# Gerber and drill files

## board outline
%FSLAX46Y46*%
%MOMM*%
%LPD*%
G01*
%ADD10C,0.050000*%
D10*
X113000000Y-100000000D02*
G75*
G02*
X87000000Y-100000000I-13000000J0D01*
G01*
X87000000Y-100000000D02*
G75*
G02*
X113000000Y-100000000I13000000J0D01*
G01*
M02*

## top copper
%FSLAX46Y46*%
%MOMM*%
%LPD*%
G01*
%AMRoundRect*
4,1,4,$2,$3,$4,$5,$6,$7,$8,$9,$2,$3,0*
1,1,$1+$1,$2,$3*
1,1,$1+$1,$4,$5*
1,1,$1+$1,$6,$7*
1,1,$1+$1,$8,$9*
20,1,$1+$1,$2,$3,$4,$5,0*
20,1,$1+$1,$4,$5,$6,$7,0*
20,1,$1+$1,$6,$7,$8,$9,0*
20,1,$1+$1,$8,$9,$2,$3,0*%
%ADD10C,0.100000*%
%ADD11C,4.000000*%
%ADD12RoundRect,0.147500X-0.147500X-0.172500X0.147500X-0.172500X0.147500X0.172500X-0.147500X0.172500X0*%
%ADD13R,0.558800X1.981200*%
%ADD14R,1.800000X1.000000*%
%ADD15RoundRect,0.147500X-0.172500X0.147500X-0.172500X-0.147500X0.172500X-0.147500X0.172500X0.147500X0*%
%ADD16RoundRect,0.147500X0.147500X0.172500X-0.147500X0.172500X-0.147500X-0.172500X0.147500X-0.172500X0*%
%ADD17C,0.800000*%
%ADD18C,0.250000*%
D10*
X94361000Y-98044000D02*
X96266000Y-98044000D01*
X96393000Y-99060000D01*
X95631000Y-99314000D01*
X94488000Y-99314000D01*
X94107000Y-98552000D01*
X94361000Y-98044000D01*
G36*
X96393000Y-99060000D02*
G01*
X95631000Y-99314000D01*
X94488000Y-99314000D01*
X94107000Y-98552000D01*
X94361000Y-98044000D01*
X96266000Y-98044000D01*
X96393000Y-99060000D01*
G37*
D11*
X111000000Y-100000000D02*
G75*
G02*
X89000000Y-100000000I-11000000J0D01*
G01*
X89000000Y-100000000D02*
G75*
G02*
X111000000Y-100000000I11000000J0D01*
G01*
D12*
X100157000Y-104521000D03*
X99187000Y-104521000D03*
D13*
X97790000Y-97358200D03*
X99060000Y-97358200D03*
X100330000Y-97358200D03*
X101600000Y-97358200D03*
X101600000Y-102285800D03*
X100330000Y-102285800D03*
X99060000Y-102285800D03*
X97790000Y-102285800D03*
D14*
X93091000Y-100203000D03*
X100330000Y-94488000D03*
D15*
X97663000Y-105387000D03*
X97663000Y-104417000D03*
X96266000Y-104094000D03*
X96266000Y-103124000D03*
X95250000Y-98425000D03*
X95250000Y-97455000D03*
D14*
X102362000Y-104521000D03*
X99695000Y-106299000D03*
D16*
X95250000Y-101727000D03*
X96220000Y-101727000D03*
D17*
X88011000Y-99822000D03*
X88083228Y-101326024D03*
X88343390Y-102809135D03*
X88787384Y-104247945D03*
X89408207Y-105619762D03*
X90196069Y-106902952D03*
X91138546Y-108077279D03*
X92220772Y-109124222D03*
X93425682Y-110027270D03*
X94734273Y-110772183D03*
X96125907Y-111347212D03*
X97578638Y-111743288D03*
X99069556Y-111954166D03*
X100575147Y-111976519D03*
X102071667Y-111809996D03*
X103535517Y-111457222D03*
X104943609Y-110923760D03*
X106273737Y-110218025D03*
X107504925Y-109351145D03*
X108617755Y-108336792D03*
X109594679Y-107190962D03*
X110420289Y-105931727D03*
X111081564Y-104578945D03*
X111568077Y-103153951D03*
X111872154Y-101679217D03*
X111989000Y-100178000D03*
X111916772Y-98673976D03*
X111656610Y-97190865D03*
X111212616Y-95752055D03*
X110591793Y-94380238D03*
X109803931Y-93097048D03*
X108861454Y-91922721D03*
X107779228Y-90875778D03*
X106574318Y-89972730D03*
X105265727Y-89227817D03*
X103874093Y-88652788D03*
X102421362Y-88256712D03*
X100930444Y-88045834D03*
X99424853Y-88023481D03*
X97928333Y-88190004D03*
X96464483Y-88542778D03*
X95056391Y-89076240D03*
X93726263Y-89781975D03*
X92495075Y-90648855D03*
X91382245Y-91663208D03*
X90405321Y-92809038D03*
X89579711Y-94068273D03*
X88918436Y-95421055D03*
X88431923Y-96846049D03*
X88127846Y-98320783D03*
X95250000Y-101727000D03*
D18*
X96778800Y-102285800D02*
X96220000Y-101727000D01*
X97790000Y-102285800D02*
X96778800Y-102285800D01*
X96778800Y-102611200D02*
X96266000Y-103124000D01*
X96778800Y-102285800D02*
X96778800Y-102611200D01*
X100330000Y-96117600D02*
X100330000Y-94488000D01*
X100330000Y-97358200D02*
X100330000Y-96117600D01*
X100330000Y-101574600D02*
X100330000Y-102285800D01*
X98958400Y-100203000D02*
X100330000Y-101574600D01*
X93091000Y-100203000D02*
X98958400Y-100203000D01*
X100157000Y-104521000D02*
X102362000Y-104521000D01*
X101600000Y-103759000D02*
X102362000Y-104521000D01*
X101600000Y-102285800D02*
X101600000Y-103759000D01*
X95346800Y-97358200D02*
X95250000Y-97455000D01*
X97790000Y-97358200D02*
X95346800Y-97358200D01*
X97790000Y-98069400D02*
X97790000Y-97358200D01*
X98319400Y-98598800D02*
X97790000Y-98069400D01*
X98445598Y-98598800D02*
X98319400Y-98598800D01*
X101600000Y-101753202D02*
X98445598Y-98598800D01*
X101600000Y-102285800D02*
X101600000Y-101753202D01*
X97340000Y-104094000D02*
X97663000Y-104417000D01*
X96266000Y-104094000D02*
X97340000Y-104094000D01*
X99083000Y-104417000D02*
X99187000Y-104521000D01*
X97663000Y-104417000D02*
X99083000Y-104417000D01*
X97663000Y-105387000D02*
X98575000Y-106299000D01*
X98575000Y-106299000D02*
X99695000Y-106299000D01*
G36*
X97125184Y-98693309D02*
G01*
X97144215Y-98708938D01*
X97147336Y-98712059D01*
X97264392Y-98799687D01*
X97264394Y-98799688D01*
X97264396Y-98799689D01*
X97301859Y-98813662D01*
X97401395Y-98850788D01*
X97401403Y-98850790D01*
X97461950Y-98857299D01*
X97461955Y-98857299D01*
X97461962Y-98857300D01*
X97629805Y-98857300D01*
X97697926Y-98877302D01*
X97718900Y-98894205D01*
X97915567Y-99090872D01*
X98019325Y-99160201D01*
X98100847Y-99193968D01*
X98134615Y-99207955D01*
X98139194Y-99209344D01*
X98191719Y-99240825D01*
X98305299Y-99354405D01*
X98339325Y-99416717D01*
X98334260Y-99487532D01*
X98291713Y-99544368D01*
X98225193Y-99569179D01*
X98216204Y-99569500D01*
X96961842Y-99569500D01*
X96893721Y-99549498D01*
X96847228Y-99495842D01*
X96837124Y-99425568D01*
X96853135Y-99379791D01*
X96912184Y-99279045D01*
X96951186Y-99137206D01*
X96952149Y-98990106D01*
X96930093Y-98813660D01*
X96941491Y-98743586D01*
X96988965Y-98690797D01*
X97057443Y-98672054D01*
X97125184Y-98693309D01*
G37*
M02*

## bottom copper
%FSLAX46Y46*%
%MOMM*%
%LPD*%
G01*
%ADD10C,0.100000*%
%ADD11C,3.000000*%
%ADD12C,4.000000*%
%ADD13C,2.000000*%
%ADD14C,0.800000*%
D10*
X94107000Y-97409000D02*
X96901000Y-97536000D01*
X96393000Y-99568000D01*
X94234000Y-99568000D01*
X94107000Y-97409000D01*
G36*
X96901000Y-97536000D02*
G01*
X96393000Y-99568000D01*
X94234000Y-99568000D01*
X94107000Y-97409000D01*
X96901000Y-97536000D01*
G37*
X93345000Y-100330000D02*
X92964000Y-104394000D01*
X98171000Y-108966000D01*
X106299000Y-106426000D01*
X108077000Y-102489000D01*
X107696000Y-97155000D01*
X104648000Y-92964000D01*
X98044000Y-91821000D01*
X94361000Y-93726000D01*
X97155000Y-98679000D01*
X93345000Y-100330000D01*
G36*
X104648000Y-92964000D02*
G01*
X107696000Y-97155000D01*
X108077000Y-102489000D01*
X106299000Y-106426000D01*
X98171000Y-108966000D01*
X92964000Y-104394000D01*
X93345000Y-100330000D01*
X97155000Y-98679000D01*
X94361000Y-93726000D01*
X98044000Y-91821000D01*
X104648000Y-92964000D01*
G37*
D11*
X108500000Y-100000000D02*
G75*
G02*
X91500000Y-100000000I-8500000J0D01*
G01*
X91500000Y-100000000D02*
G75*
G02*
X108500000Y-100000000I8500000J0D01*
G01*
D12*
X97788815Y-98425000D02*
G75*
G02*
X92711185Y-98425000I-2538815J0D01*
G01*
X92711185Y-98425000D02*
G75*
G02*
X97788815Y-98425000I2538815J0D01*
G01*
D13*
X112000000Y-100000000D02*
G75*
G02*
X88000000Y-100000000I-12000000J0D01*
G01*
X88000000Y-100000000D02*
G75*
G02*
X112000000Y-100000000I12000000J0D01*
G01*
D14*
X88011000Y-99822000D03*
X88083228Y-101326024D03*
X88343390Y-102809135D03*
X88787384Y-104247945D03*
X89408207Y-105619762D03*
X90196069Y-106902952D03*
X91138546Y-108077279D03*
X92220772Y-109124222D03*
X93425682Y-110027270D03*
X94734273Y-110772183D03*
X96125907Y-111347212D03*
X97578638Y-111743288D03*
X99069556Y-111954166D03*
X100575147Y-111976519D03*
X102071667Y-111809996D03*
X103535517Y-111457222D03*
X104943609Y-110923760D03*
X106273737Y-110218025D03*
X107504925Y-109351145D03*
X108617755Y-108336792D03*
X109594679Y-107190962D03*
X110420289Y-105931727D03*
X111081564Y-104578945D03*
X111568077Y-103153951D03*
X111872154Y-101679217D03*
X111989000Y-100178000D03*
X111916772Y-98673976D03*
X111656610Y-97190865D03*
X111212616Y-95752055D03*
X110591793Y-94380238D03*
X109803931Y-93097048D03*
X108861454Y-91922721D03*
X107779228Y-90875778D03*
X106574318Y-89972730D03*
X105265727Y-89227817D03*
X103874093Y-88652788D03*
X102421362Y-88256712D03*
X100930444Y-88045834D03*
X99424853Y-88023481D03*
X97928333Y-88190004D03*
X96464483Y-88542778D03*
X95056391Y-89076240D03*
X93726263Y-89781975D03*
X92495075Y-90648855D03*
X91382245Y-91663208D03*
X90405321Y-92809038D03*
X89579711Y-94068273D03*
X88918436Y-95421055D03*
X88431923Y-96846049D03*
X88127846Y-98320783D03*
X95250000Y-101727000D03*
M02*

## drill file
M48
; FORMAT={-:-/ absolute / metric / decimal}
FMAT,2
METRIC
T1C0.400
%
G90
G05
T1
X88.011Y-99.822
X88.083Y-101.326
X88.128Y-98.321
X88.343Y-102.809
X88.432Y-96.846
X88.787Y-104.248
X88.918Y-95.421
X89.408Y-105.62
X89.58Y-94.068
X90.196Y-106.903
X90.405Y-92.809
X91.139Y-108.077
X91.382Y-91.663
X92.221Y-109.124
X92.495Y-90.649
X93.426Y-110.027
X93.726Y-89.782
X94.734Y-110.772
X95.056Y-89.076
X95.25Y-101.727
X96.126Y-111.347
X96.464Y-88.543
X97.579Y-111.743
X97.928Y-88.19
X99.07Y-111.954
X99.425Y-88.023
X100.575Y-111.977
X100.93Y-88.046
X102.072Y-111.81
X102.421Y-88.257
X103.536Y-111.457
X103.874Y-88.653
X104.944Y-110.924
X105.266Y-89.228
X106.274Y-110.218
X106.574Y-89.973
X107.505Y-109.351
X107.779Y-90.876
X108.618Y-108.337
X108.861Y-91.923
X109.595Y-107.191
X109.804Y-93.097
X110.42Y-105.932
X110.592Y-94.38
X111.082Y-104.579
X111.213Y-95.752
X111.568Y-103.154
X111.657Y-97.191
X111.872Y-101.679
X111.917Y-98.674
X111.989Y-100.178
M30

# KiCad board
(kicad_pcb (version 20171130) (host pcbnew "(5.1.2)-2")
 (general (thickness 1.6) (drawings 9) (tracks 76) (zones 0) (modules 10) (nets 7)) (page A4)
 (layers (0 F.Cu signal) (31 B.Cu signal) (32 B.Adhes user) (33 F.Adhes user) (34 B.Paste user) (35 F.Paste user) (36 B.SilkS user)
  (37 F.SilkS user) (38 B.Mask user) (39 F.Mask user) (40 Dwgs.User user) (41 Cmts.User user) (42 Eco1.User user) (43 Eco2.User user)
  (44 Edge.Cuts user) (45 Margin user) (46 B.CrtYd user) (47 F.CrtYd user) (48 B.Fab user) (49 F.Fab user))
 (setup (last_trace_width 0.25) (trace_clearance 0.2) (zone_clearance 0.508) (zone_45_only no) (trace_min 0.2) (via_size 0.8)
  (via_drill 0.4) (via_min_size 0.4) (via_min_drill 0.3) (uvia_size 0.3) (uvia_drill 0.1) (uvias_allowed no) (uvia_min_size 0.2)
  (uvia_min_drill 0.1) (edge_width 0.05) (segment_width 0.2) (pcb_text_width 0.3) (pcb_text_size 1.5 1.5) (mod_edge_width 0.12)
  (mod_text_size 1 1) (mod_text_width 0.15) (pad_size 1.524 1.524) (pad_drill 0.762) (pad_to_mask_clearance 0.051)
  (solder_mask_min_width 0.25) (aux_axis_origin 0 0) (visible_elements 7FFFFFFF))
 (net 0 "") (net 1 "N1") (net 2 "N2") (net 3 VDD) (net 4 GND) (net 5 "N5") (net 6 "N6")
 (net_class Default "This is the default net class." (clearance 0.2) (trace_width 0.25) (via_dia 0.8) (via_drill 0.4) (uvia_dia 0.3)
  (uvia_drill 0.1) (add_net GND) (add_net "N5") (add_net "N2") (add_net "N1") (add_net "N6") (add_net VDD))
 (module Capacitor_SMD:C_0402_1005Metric (layer F.Cu) (at 99.672 104.521)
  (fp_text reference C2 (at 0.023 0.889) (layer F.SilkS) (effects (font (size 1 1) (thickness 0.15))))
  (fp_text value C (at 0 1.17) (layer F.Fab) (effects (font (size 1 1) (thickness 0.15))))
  (pad 2 smd roundrect (at 0.485 0) (size 0.59 0.64) (layers F.Cu F.Paste F.Mask) (roundrect_rratio 0.25) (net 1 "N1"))
  (pad 1 smd roundrect (at -0.485 0) (size 0.59 0.64) (layers F.Cu F.Paste F.Mask) (roundrect_rratio 0.25) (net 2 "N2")))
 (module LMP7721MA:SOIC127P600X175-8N (layer F.Cu) (at 99.695 99.822 90)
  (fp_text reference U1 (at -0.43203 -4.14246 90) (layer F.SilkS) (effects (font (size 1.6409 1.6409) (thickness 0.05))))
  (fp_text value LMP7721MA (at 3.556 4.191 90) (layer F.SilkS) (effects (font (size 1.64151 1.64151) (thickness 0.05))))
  (pad 8 smd rect (at 2.4638 -1.905 90) (size 1.9812 0.5588) (layers F.Cu F.Paste F.Mask) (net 1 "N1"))
  (pad 7 smd rect (at 2.4638 -0.635 90) (size 1.9812 0.5588) (layers F.Cu F.Paste F.Mask))
  (pad 6 smd rect (at 2.4638 0.635 90) (size 1.9812 0.5588) (layers F.Cu F.Paste F.Mask) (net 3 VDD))
  (pad 5 smd rect (at 2.4638 1.905 90) (size 1.9812 0.5588) (layers F.Cu F.Paste F.Mask))
  (pad 4 smd rect (at -2.4638 1.905 90) (size 1.9812 0.5588) (layers F.Cu F.Paste F.Mask) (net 1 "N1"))
  (pad 3 smd rect (at -2.4638 0.635 90) (size 1.9812 0.5588) (layers F.Cu F.Paste F.Mask) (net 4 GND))
  (pad 2 smd rect (at -2.4638 -0.635 90) (size 1.9812 0.5588) (layers F.Cu F.Paste F.Mask))
  (pad 1 smd rect (at -2.4638 -1.905 90) (size 1.9812 0.5588) (layers F.Cu F.Paste F.Mask) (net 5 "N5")))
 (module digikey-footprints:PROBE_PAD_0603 (layer F.Cu) (at 93.091 100.203)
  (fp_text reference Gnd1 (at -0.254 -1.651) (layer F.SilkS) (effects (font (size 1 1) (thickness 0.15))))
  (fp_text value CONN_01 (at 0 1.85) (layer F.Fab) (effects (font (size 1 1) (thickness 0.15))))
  (pad 1 smd rect (at 0 0) (size 1.8 1) (layers F.Cu F.Paste F.Mask) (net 4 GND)))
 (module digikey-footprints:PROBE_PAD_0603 (layer F.Cu) (at 100.33 94.488)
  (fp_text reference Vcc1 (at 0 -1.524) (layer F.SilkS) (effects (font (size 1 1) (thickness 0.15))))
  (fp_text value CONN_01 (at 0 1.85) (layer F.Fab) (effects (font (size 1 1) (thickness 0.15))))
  (pad 1 smd rect (at 0 0) (size 1.8 1) (layers F.Cu F.Paste F.Mask) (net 3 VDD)))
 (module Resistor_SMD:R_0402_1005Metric (layer F.Cu) (at 97.663 104.902 270)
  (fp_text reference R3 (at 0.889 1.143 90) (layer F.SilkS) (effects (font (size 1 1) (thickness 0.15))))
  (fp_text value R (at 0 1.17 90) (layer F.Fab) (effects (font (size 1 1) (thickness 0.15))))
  (pad 2 smd roundrect (at 0.485 0 270) (size 0.59 0.64) (layers F.Cu F.Paste F.Mask) (roundrect_rratio 0.25) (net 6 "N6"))
  (pad 1 smd roundrect (at -0.485 0 270) (size 0.59 0.64) (layers F.Cu F.Paste F.Mask) (roundrect_rratio 0.25) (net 2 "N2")))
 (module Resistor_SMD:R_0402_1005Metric (layer F.Cu) (at 96.266 103.609 270)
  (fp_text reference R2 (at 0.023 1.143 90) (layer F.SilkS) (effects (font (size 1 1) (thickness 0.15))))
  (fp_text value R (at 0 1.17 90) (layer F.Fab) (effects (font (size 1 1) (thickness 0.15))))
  (pad 2 smd roundrect (at 0.485 0 270) (size 0.59 0.64) (layers F.Cu F.Paste F.Mask) (roundrect_rratio 0.25) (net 2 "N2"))
  (pad 1 smd roundrect (at -0.485 0 270) (size 0.59 0.64) (layers F.Cu F.Paste F.Mask) (roundrect_rratio 0.25) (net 5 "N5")))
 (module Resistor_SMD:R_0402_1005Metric (layer F.Cu) (at 95.25 97.94 270)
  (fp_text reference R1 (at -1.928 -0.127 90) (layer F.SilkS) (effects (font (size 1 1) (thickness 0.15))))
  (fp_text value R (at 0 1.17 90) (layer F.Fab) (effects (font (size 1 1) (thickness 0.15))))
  (pad 2 smd roundrect (at 0.485 0 270) (size 0.59 0.64) (layers F.Cu F.Paste F.Mask) (roundrect_rratio 0.25))
  (pad 1 smd roundrect (at -0.485 0 270) (size 0.59 0.64) (layers F.Cu F.Paste F.Mask) (roundrect_rratio 0.25) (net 1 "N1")))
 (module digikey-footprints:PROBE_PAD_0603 (layer F.Cu) (at 102.362 104.521)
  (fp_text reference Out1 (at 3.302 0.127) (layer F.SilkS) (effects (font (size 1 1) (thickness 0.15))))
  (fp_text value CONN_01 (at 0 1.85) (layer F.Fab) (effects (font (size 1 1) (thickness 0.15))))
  (pad 1 smd rect (at 0 0) (size 1.8 1) (layers F.Cu F.Paste F.Mask) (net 1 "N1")))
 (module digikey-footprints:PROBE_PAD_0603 (layer F.Cu) (at 99.695 106.299)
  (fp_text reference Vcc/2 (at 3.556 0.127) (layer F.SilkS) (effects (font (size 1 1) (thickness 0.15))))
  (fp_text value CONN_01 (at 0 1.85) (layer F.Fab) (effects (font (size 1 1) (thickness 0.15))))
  (pad 1 smd rect (at 0 0) (size 1.8 1) (layers F.Cu F.Paste F.Mask) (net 6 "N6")))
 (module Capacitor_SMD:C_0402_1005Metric (layer F.Cu) (at 95.735 101.727 180)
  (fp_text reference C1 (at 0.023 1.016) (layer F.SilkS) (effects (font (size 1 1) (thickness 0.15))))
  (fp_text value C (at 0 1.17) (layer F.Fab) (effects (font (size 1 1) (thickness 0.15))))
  (pad 2 smd roundrect (at 0.485 0 180) (size 0.59 0.64) (layers F.Cu F.Paste F.Mask) (roundrect_rratio 0.25))
  (pad 1 smd roundrect (at -0.485 0 180) (size 0.59 0.64) (layers F.Cu F.Paste F.Mask) (roundrect_rratio 0.25) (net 5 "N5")))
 (gr_poly
  (pts (xy 94.361 98.044) (xy 96.266 98.044) (xy 96.393 99.06) (xy 95.631 99.314) (xy 94.488 99.314) (xy 94.107 98.552)) (layer F.Cu)
  (width 0.1))
 (gr_circle (center 100 100) (end 111 100) (layer F.Cu) (width 4))
 (gr_circle (center 100 100) (end 113 100) (layer Edge.Cuts) (width 0.05))
 (gr_poly (pts (xy 94.107 97.409) (xy 96.901 97.536) (xy 96.393 99.568) (xy 94.234 99.568)) (layer B.Cu) (width 0.1))
 (gr_poly
  (pts (xy 93.345 100.33) (xy 92.964 104.394) (xy 98.171 108.966) (xy 106.299 106.426) (xy 108.077 102.489) (xy 107.696 97.155)
   (xy 104.648 92.964) (xy 98.044 91.821) (xy 94.361 93.726) (xy 97.155 98.679))
  (layer B.Cu) (width 0.1))
 (gr_circle (center 100 100) (end 108.5 100) (layer B.Cu) (width 3))
 (gr_circle (center 95.25 98.425) (end 97.788815 98.425) (layer B.Cu) (width 4))
 (gr_circle (center 100 100) (end 112 100) (layer B.Cu) (width 2))
 (via (at 88.011 99.822) (size 0.8) (drill 0.4) (layers F.Cu B.Cu) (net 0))
 (via (at 88.083228 101.326024) (size 0.8) (drill 0.4) (layers F.Cu B.Cu) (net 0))
 (via (at 88.34339 102.809135) (size 0.8) (drill 0.4) (layers F.Cu B.Cu) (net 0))
 (via (at 88.787384 104.247945) (size 0.8) (drill 0.4) (layers F.Cu B.Cu) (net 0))
 (via (at 89.408207 105.619762) (size 0.8) (drill 0.4) (layers F.Cu B.Cu) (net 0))
 (via (at 90.196069 106.902952) (size 0.8) (drill 0.4) (layers F.Cu B.Cu) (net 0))
 (via (at 91.138546 108.077279) (size 0.8) (drill 0.4) (layers F.Cu B.Cu) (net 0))
 (via (at 92.220772 109.124222) (size 0.8) (drill 0.4) (layers F.Cu B.Cu) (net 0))
 (via (at 93.425682 110.02727) (size 0.8) (drill 0.4) (layers F.Cu B.Cu) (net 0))
 (via (at 94.734273 110.772183) (size 0.8) (drill 0.4) (layers F.Cu B.Cu) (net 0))
 (via (at 96.125907 111.347212) (size 0.8) (drill 0.4) (layers F.Cu B.Cu) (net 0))
 (via (at 97.578638 111.743288) (size 0.8) (drill 0.4) (layers F.Cu B.Cu) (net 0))
 (via (at 99.069556 111.954166) (size 0.8) (drill 0.4) (layers F.Cu B.Cu) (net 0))
 (via (at 100.575147 111.976519) (size 0.8) (drill 0.4) (layers F.Cu B.Cu) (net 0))
 (via (at 102.071667 111.809996) (size 0.8) (drill 0.4) (layers F.Cu B.Cu) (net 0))
 (via (at 103.535517 111.457222) (size 0.8) (drill 0.4) (layers F.Cu B.Cu) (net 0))
 (via (at 104.943609 110.92376) (size 0.8) (drill 0.4) (layers F.Cu B.Cu) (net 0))
 (via (at 106.273737 110.218025) (size 0.8) (drill 0.4) (layers F.Cu B.Cu) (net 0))
 (via (at 107.504925 109.351145) (size 0.8) (drill 0.4) (layers F.Cu B.Cu) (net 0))
 (via (at 108.617755 108.336792) (size 0.8) (drill 0.4) (layers F.Cu B.Cu) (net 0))
 (via (at 109.594679 107.190962) (size 0.8) (drill 0.4) (layers F.Cu B.Cu) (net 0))
 (via (at 110.420289 105.931727) (size 0.8) (drill 0.4) (layers F.Cu B.Cu) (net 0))
 (via (at 111.081564 104.578945) (size 0.8) (drill 0.4) (layers F.Cu B.Cu) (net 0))
 (via (at 111.568077 103.153951) (size 0.8) (drill 0.4) (layers F.Cu B.Cu) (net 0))
 (via (at 111.872154 101.679217) (size 0.8) (drill 0.4) (layers F.Cu B.Cu) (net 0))
 (via (at 111.989 100.178) (size 0.8) (drill 0.4) (layers F.Cu B.Cu) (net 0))
 (via (at 111.916772 98.673976) (size 0.8) (drill 0.4) (layers F.Cu B.Cu) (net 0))
 (via (at 111.65661 97.190865) (size 0.8) (drill 0.4) (layers F.Cu B.Cu) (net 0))
 (via (at 111.212616 95.752055) (size 0.8) (drill 0.4) (layers F.Cu B.Cu) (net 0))
 (via (at 110.591793 94.380238) (size 0.8) (drill 0.4) (layers F.Cu B.Cu) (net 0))
 (via (at 109.803931 93.097048) (size 0.8) (drill 0.4) (layers F.Cu B.Cu) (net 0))
 (via (at 108.861454 91.922721) (size 0.8) (drill 0.4) (layers F.Cu B.Cu) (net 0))
 (via (at 107.779228 90.875778) (size 0.8) (drill 0.4) (layers F.Cu B.Cu) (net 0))
 (via (at 106.574318 89.97273) (size 0.8) (drill 0.4) (layers F.Cu B.Cu) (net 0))
 (via (at 105.265727 89.227817) (size 0.8) (drill 0.4) (layers F.Cu B.Cu) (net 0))
 (via (at 103.874093 88.652788) (size 0.8) (drill 0.4) (layers F.Cu B.Cu) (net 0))
 (via (at 102.421362 88.256712) (size 0.8) (drill 0.4) (layers F.Cu B.Cu) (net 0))
 (via (at 100.930444 88.045834) (size 0.8) (drill 0.4) (layers F.Cu B.Cu) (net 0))
 (via (at 99.424853 88.023481) (size 0.8) (drill 0.4) (layers F.Cu B.Cu) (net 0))
 (via (at 97.928333 88.190004) (size 0.8) (drill 0.4) (layers F.Cu B.Cu) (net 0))
 (via (at 96.464483 88.542778) (size 0.8) (drill 0.4) (layers F.Cu B.Cu) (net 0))
 (via (at 95.056391 89.07624) (size 0.8) (drill 0.4) (layers F.Cu B.Cu) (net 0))
 (via (at 93.726263 89.781975) (size 0.8) (drill 0.4) (layers F.Cu B.Cu) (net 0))
 (via (at 92.495075 90.648855) (size 0.8) (drill 0.4) (layers F.Cu B.Cu) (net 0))
 (via (at 91.382245 91.663208) (size 0.8) (drill 0.4) (layers F.Cu B.Cu) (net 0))
 (via (at 90.405321 92.809038) (size 0.8) (drill 0.4) (layers F.Cu B.Cu) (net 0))
 (via (at 89.579711 94.068273) (size 0.8) (drill 0.4) (layers F.Cu B.Cu) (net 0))
 (via (at 88.918436 95.421055) (size 0.8) (drill 0.4) (layers F.Cu B.Cu) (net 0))
 (via (at 88.431923 96.846049) (size 0.8) (drill 0.4) (layers F.Cu B.Cu) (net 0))
 (via (at 88.127846 98.320783) (size 0.8) (drill 0.4) (layers F.Cu B.Cu) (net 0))
 (via (at 95.25 101.727) (size 0.8) (drill 0.4) (layers F.Cu B.Cu) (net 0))
 (segment (start 96.7788 102.2858) (end 96.22 101.727) (width 0.25) (layer F.Cu) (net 5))
 (segment (start 97.79 102.2858) (end 96.7788 102.2858) (width 0.25) (layer F.Cu) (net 5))
 (segment (start 96.7788 102.6112) (end 96.266 103.124) (width 0.25) (layer F.Cu) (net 5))
 (segment (start 96.7788 102.2858) (end 96.7788 102.6112) (width 0.25) (layer F.Cu) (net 5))
 (segment (start 100.33 96.1176) (end 100.33 94.488) (width 0.25) (layer F.Cu) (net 3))
 (segment (start 100.33 97.3582) (end 100.33 96.1176) (width 0.25) (layer F.Cu) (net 3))
 (segment (start 100.33 101.5746) (end 100.33 102.2858) (width 0.25) (layer F.Cu) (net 4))
 (segment (start 98.9584 100.203) (end 100.33 101.5746) (width 0.25) (layer F.Cu) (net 4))
 (segment (start 93.091 100.203) (end 98.9584 100.203) (width 0.25) (layer F.Cu) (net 4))
 (segment (start 100.157 104.521) (end 102.362 104.521) (width 0.25) (layer F.Cu) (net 1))
 (segment (start 101.6 103.759) (end 102.362 104.521) (width 0.25) (layer F.Cu) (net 1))
 (segment (start 101.6 102.2858) (end 101.6 103.759) (width 0.25) (layer F.Cu) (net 1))
 (segment (start 95.3468 97.3582) (end 95.25 97.455) (width 0.25) (layer F.Cu) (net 1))
 (segment (start 97.79 97.3582) (end 95.3468 97.3582) (width 0.25) (layer F.Cu) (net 1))
 (segment (start 97.79 98.0694) (end 97.79 97.3582) (width 0.25) (layer F.Cu) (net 1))
 (segment (start 98.3194 98.5988) (end 97.79 98.0694) (width 0.25) (layer F.Cu) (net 1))
 (segment (start 98.445598 98.5988) (end 98.3194 98.5988) (width 0.25) (layer F.Cu) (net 1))
 (segment (start 101.6 101.753202) (end 98.445598 98.5988) (width 0.25) (layer F.Cu) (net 1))
 (segment (start 101.6 102.2858) (end 101.6 101.753202) (width 0.25) (layer F.Cu) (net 1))
 (segment (start 97.34 104.094) (end 97.663 104.417) (width 0.25) (layer F.Cu) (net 2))
 (segment (start 96.266 104.094) (end 97.34 104.094) (width 0.25) (layer F.Cu) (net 2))
 (segment (start 99.083 104.417) (end 99.187 104.521) (width 0.25) (layer F.Cu) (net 2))
 (segment (start 97.663 104.417) (end 99.083 104.417) (width 0.25) (layer F.Cu) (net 2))
 (segment (start 97.663 105.387) (end 98.575 106.299) (width 0.25) (layer F.Cu) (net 6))
 (segment (start 98.575 106.299) (end 99.695 106.299) (width 0.25) (layer F.Cu) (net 6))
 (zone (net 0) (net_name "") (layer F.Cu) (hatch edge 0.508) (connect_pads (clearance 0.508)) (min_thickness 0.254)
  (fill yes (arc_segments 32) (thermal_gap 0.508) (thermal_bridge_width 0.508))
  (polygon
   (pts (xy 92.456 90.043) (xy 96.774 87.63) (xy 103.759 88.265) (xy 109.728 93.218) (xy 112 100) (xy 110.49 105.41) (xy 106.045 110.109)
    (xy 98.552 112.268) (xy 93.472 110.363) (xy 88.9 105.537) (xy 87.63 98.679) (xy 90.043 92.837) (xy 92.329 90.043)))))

